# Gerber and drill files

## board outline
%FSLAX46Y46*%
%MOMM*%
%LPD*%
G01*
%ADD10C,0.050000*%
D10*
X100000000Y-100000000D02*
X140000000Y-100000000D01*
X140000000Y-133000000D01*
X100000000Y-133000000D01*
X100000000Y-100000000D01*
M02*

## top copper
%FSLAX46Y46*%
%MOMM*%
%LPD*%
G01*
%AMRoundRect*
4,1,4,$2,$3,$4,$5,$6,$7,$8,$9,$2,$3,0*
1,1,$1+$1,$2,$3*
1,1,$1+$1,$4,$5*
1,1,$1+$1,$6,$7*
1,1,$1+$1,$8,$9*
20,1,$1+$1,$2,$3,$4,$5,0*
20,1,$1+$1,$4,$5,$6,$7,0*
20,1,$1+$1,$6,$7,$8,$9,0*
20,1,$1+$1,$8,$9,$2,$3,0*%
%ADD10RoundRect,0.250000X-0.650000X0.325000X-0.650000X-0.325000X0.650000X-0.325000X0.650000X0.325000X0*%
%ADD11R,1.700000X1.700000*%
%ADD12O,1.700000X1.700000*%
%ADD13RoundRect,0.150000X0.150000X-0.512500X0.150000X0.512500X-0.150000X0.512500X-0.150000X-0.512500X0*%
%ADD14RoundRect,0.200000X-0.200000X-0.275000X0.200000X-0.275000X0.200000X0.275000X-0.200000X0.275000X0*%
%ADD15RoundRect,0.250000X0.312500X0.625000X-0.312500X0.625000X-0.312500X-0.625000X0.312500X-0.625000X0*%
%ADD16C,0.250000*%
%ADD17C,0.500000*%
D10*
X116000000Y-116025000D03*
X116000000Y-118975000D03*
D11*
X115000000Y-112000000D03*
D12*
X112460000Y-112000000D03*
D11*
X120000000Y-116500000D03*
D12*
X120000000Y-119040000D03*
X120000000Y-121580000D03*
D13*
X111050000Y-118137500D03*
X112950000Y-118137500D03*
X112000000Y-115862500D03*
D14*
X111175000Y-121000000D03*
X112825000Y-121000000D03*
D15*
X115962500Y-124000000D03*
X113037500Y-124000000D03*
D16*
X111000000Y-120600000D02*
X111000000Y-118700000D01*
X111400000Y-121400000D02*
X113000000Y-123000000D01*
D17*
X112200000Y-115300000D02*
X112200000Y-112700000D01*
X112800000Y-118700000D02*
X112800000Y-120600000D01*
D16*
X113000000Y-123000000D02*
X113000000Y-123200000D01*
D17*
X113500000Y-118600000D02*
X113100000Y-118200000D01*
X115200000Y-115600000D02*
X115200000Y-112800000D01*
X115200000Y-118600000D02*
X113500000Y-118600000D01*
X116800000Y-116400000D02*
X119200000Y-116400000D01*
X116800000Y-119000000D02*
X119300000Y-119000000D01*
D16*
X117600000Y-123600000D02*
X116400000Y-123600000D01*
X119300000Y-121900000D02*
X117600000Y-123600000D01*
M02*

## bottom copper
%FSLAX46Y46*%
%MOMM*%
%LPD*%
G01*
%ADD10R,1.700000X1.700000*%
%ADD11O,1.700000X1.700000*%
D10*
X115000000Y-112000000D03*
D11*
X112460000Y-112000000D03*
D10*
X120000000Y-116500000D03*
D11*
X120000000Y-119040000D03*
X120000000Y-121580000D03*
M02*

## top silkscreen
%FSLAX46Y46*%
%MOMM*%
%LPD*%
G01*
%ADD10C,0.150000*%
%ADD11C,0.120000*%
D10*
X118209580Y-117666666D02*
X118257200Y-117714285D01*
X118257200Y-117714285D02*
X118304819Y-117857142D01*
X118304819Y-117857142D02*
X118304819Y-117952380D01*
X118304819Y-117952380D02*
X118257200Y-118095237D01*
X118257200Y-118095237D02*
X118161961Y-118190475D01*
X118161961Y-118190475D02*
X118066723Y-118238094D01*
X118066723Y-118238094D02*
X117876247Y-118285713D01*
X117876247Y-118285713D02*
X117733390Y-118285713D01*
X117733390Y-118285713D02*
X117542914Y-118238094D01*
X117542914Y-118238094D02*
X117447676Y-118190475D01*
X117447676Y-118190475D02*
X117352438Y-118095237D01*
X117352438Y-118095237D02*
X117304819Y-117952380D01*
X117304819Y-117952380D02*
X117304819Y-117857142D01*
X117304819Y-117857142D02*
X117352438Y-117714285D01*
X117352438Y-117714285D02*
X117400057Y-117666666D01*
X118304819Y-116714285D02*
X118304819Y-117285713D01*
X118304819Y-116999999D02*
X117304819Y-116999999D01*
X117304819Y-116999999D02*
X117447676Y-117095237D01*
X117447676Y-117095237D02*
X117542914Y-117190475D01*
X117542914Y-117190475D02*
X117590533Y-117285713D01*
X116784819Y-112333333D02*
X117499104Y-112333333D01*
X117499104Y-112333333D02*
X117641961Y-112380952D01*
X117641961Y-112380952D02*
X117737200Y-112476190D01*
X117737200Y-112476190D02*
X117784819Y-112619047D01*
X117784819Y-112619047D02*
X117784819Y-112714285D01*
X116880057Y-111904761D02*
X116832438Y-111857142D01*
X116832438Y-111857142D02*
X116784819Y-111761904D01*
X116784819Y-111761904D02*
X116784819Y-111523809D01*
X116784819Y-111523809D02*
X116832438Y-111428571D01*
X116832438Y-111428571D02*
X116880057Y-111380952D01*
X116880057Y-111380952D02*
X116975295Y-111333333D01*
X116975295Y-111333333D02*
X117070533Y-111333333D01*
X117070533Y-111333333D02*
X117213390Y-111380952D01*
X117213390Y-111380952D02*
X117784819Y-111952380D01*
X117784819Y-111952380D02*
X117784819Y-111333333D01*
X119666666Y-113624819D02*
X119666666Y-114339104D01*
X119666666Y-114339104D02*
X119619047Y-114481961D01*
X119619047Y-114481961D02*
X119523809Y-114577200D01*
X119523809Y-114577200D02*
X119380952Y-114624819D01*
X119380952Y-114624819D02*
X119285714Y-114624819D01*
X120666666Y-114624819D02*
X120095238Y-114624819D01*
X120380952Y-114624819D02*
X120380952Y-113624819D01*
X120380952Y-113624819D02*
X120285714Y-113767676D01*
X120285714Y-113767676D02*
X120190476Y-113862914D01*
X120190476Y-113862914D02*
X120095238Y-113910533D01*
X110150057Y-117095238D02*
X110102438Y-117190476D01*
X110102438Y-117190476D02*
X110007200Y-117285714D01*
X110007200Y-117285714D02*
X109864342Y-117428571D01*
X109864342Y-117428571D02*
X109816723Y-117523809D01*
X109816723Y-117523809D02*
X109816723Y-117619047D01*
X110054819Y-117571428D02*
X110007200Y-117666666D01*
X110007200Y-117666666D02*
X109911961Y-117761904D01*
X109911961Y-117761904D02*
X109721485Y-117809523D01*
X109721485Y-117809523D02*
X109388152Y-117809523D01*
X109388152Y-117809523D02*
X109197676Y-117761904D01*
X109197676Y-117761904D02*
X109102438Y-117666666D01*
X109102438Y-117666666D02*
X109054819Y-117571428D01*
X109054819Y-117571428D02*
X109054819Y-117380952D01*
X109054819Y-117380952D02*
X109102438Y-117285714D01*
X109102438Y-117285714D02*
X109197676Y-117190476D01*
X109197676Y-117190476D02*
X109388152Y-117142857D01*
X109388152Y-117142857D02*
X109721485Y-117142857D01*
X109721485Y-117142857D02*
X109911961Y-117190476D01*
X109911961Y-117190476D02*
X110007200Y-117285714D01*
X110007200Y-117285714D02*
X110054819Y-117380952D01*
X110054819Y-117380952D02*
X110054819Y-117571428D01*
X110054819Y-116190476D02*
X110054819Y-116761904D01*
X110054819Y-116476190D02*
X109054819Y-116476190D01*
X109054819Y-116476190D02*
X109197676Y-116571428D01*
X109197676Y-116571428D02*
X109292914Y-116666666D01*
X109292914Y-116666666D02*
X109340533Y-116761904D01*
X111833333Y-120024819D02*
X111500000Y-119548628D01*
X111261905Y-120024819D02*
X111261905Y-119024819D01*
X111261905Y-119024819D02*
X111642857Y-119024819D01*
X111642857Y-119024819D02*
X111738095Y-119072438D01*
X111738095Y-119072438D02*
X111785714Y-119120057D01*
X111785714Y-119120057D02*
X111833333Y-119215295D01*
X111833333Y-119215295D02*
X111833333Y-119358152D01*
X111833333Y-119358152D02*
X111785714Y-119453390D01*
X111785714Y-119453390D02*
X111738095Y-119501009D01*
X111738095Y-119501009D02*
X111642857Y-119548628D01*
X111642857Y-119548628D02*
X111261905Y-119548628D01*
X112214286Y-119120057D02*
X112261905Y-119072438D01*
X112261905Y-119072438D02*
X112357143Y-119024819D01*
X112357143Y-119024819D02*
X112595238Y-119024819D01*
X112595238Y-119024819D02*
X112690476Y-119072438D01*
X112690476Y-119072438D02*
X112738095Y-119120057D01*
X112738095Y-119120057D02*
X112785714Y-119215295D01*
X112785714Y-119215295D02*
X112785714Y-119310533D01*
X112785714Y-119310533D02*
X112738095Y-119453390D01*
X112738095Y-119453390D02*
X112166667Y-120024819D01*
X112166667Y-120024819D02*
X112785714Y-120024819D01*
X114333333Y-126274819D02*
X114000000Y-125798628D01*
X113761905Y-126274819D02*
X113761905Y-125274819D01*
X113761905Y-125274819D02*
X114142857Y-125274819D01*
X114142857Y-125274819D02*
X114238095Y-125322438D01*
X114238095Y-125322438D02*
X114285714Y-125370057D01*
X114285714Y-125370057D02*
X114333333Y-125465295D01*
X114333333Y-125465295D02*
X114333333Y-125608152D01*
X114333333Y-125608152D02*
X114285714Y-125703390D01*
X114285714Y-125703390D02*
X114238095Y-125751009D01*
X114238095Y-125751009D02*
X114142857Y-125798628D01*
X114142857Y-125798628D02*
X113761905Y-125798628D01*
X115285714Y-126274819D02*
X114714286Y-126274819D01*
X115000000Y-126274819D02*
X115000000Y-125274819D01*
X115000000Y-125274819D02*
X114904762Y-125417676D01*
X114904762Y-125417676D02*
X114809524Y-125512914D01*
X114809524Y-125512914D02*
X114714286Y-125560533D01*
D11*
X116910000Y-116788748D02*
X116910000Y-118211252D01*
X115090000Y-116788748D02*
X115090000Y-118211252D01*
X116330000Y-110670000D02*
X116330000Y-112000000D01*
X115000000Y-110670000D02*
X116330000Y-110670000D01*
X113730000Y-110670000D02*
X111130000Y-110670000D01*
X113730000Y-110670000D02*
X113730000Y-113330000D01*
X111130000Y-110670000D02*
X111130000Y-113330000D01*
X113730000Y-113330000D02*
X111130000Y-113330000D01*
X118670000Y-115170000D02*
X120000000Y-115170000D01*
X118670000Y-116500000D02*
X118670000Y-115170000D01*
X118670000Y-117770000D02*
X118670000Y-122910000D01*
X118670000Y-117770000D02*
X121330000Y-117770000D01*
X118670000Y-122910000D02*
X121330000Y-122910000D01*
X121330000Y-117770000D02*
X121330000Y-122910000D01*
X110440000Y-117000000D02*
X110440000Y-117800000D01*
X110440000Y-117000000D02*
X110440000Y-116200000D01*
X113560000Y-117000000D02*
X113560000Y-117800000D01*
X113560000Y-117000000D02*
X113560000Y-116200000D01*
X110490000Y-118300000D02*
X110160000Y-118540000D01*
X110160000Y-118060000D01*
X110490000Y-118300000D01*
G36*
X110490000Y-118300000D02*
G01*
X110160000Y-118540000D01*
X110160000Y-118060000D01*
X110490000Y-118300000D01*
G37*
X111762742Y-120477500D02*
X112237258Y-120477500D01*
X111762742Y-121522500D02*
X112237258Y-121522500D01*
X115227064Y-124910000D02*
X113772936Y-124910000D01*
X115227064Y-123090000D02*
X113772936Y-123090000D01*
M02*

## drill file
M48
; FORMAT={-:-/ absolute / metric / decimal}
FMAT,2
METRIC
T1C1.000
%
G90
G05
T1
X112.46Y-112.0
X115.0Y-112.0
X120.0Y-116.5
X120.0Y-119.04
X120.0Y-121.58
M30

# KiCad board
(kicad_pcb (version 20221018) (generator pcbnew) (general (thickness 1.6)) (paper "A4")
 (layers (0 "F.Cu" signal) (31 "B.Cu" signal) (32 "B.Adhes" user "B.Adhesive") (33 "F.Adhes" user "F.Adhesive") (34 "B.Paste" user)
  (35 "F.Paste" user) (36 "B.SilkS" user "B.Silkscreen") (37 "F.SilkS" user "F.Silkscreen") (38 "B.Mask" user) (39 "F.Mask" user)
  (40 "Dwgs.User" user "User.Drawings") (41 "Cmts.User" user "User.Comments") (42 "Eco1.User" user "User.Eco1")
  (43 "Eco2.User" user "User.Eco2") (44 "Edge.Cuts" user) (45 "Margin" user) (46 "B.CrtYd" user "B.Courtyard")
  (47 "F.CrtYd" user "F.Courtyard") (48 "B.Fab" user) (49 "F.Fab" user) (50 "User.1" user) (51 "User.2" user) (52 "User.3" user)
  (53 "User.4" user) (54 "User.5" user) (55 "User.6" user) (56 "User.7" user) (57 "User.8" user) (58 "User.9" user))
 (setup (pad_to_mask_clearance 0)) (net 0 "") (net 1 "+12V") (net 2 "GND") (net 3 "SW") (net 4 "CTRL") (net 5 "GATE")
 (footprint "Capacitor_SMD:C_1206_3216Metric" (layer "F.Cu") (at 116 117.5 -90)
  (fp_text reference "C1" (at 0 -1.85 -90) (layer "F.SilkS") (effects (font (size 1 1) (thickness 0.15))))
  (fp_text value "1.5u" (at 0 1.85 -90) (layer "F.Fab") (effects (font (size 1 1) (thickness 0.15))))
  (fp_line (start -0.711252 -0.91) (end 0.711252 -0.91) (stroke (width 0.12) (type solid)) (layer "F.SilkS"))
  (fp_line (start -0.711252 0.91) (end 0.711252 0.91) (stroke (width 0.12) (type solid)) (layer "F.SilkS"))
  (pad "1" smd roundrect (at -1.475 0 270) (size 1.15 1.8) (layers "F.Cu" "F.Paste" "F.Mask") (roundrect_rratio 0.217391) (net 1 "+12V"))
  (pad "2" smd roundrect (at 1.475 0 270) (size 1.15 1.8) (layers "F.Cu" "F.Paste" "F.Mask") (roundrect_rratio 0.217391) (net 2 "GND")))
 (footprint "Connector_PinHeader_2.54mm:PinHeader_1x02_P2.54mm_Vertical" (layer "F.Cu") (at 115 112 -90)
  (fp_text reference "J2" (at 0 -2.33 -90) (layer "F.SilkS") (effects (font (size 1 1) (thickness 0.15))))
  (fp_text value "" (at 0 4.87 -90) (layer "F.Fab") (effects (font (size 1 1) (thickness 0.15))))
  (fp_line (start -1.33 -1.33) (end 0 -1.33) (stroke (width 0.12) (type solid)) (layer "F.SilkS"))
  (fp_line (start -1.33 0) (end -1.33 -1.33) (stroke (width 0.12) (type solid)) (layer "F.SilkS"))
  (fp_line (start -1.33 1.27) (end -1.33 3.87) (stroke (width 0.12) (type solid)) (layer "F.SilkS"))
  (fp_line (start -1.33 1.27) (end 1.33 1.27) (stroke (width 0.12) (type solid)) (layer "F.SilkS"))
  (fp_line (start -1.33 3.87) (end 1.33 3.87) (stroke (width 0.12) (type solid)) (layer "F.SilkS"))
  (fp_line (start 1.33 1.27) (end 1.33 3.87) (stroke (width 0.12) (type solid)) (layer "F.SilkS"))
  (pad "1" thru_hole rect (at 0 0 270) (size 1.7 1.7) (drill 1) (layers "*.Cu" "*.Mask") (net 1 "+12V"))
  (pad "2" thru_hole oval (at 0 2.54 270) (size 1.7 1.7) (drill 1) (layers "*.Cu" "*.Mask") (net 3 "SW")))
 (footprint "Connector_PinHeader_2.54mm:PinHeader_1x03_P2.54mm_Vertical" (layer "F.Cu") (at 120 116.5)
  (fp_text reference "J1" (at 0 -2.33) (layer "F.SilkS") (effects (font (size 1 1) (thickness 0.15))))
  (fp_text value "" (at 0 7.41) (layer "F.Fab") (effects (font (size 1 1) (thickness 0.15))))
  (fp_line (start -1.33 -1.33) (end 0 -1.33) (stroke (width 0.12) (type solid)) (layer "F.SilkS"))
  (fp_line (start -1.33 0) (end -1.33 -1.33) (stroke (width 0.12) (type solid)) (layer "F.SilkS"))
  (fp_line (start -1.33 1.27) (end -1.33 6.41) (stroke (width 0.12) (type solid)) (layer "F.SilkS"))
  (fp_line (start -1.33 1.27) (end 1.33 1.27) (stroke (width 0.12) (type solid)) (layer "F.SilkS"))
  (fp_line (start -1.33 6.41) (end 1.33 6.41) (stroke (width 0.12) (type solid)) (layer "F.SilkS"))
  (fp_line (start 1.33 1.27) (end 1.33 6.41) (stroke (width 0.12) (type solid)) (layer "F.SilkS"))
  (pad "1" thru_hole rect (at 0 0) (size 1.7 1.7) (drill 1) (layers "*.Cu" "*.Mask") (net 1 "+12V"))
  (pad "2" thru_hole oval (at 0 2.54) (size 1.7 1.7) (drill 1) (layers "*.Cu" "*.Mask") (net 2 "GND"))
  (pad "3" thru_hole oval (at 0 5.08) (size 1.7 1.7) (drill 1) (layers "*.Cu" "*.Mask") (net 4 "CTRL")))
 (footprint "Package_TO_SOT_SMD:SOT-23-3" (layer "F.Cu") (at 112 117 90)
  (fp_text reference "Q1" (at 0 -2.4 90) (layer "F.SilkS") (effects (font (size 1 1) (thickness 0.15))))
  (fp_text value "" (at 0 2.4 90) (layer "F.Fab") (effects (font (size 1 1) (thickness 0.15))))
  (fp_line (start 0 -1.56) (end -0.8 -1.56) (stroke (width 0.12) (type solid)) (layer "F.SilkS"))
  (fp_line (start 0 -1.56) (end 0.8 -1.56) (stroke (width 0.12) (type solid)) (layer "F.SilkS"))
  (fp_line (start 0 1.56) (end -0.8 1.56) (stroke (width 0.12) (type solid)) (layer "F.SilkS"))
  (fp_line (start 0 1.56) (end 0.8 1.56) (stroke (width 0.12) (type solid)) (layer "F.SilkS"))
  (fp_poly
   (pts (xy -1.3 -1.51) (xy -1.54 -1.84) (xy -1.06 -1.84) (xy -1.3 -1.51)) (stroke (width 0.12) (type solid)) (fill solid) (layer "F.SilkS"))
  (pad "1" smd roundrect (at -1.1375 -0.95 90) (size 1.325 0.6) (layers "F.Cu" "F.Paste" "F.Mask") (roundrect_rratio 0.25) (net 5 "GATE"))
  (pad "2" smd roundrect (at -1.1375 0.95 90) (size 1.325 0.6) (layers "F.Cu" "F.Paste" "F.Mask") (roundrect_rratio 0.25) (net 2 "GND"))
  (pad "3" smd roundrect (at 1.1375 0 90) (size 1.325 0.6) (layers "F.Cu" "F.Paste" "F.Mask") (roundrect_rratio 0.25) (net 3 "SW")))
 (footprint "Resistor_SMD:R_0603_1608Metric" (layer "F.Cu") (at 112 121)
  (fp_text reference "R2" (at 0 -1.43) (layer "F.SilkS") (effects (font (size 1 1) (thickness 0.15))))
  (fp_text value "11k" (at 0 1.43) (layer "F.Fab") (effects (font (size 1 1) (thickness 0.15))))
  (fp_line (start -0.237258 -0.5225) (end 0.237258 -0.5225) (stroke (width 0.12) (type solid)) (layer "F.SilkS"))
  (fp_line (start -0.237258 0.5225) (end 0.237258 0.5225) (stroke (width 0.12) (type solid)) (layer "F.SilkS"))
  (pad "1" smd roundrect (at -0.825 0) (size 0.8 0.95) (layers "F.Cu" "F.Paste" "F.Mask") (roundrect_rratio 0.25) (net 5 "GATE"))
  (pad "2" smd roundrect (at 0.825 0) (size 0.8 0.95) (layers "F.Cu" "F.Paste" "F.Mask") (roundrect_rratio 0.25) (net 2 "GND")))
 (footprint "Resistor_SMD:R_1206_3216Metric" (layer "F.Cu") (at 114.5 124 180)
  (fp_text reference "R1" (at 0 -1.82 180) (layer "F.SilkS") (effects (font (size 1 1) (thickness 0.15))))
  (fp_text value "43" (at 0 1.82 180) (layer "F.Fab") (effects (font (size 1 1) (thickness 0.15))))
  (fp_line (start -0.727064 -0.91) (end 0.727064 -0.91) (stroke (width 0.12) (type solid)) (layer "F.SilkS"))
  (fp_line (start -0.727064 0.91) (end 0.727064 0.91) (stroke (width 0.12) (type solid)) (layer "F.SilkS"))
  (pad "1" smd roundrect (at -1.4625 0 180) (size 1.125 1.75) (layers "F.Cu" "F.Paste" "F.Mask") (roundrect_rratio 0.222222) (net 4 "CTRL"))
  (pad "2" smd roundrect (at 1.4625 0 180) (size 1.125 1.75) (layers "F.Cu" "F.Paste" "F.Mask") (roundrect_rratio 0.222222) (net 5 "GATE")))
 (gr_rect (start 100 100) (end 140 133) (stroke (width 0.05) (type default)) (fill none) (layer "Edge.Cuts"))
 (segment (start 111 120.6) (end 111 118.7) (width 0.25) (layer "F.Cu") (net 5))
 (segment (start 111.4 121.4) (end 113 123) (width 0.25) (layer "F.Cu") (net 5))
 (segment (start 112.2 115.3) (end 112.2 112.7) (width 0.5) (layer "F.Cu") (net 3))
 (segment (start 112.8 118.7) (end 112.8 120.6) (width 0.5) (layer "F.Cu") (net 2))
 (segment (start 113 123) (end 113 123.2) (width 0.25) (layer "F.Cu") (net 5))
 (segment (start 113.5 118.6) (end 113.1 118.2) (width 0.5) (layer "F.Cu") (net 2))
 (segment (start 115.2 115.6) (end 115.2 112.8) (width 0.5) (layer "F.Cu") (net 1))
 (segment (start 115.2 118.6) (end 113.5 118.6) (width 0.5) (layer "F.Cu") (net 2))
 (segment (start 116.8 116.4) (end 119.2 116.4) (width 0.5) (layer "F.Cu") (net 1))
 (segment (start 116.8 119) (end 119.3 119) (width 0.5) (layer "F.Cu") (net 2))
 (segment (start 117.6 123.6) (end 116.4 123.6) (width 0.25) (layer "F.Cu") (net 4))
 (segment (start 119.3 121.9) (end 117.6 123.6) (width 0.25) (layer "F.Cu") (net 4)))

